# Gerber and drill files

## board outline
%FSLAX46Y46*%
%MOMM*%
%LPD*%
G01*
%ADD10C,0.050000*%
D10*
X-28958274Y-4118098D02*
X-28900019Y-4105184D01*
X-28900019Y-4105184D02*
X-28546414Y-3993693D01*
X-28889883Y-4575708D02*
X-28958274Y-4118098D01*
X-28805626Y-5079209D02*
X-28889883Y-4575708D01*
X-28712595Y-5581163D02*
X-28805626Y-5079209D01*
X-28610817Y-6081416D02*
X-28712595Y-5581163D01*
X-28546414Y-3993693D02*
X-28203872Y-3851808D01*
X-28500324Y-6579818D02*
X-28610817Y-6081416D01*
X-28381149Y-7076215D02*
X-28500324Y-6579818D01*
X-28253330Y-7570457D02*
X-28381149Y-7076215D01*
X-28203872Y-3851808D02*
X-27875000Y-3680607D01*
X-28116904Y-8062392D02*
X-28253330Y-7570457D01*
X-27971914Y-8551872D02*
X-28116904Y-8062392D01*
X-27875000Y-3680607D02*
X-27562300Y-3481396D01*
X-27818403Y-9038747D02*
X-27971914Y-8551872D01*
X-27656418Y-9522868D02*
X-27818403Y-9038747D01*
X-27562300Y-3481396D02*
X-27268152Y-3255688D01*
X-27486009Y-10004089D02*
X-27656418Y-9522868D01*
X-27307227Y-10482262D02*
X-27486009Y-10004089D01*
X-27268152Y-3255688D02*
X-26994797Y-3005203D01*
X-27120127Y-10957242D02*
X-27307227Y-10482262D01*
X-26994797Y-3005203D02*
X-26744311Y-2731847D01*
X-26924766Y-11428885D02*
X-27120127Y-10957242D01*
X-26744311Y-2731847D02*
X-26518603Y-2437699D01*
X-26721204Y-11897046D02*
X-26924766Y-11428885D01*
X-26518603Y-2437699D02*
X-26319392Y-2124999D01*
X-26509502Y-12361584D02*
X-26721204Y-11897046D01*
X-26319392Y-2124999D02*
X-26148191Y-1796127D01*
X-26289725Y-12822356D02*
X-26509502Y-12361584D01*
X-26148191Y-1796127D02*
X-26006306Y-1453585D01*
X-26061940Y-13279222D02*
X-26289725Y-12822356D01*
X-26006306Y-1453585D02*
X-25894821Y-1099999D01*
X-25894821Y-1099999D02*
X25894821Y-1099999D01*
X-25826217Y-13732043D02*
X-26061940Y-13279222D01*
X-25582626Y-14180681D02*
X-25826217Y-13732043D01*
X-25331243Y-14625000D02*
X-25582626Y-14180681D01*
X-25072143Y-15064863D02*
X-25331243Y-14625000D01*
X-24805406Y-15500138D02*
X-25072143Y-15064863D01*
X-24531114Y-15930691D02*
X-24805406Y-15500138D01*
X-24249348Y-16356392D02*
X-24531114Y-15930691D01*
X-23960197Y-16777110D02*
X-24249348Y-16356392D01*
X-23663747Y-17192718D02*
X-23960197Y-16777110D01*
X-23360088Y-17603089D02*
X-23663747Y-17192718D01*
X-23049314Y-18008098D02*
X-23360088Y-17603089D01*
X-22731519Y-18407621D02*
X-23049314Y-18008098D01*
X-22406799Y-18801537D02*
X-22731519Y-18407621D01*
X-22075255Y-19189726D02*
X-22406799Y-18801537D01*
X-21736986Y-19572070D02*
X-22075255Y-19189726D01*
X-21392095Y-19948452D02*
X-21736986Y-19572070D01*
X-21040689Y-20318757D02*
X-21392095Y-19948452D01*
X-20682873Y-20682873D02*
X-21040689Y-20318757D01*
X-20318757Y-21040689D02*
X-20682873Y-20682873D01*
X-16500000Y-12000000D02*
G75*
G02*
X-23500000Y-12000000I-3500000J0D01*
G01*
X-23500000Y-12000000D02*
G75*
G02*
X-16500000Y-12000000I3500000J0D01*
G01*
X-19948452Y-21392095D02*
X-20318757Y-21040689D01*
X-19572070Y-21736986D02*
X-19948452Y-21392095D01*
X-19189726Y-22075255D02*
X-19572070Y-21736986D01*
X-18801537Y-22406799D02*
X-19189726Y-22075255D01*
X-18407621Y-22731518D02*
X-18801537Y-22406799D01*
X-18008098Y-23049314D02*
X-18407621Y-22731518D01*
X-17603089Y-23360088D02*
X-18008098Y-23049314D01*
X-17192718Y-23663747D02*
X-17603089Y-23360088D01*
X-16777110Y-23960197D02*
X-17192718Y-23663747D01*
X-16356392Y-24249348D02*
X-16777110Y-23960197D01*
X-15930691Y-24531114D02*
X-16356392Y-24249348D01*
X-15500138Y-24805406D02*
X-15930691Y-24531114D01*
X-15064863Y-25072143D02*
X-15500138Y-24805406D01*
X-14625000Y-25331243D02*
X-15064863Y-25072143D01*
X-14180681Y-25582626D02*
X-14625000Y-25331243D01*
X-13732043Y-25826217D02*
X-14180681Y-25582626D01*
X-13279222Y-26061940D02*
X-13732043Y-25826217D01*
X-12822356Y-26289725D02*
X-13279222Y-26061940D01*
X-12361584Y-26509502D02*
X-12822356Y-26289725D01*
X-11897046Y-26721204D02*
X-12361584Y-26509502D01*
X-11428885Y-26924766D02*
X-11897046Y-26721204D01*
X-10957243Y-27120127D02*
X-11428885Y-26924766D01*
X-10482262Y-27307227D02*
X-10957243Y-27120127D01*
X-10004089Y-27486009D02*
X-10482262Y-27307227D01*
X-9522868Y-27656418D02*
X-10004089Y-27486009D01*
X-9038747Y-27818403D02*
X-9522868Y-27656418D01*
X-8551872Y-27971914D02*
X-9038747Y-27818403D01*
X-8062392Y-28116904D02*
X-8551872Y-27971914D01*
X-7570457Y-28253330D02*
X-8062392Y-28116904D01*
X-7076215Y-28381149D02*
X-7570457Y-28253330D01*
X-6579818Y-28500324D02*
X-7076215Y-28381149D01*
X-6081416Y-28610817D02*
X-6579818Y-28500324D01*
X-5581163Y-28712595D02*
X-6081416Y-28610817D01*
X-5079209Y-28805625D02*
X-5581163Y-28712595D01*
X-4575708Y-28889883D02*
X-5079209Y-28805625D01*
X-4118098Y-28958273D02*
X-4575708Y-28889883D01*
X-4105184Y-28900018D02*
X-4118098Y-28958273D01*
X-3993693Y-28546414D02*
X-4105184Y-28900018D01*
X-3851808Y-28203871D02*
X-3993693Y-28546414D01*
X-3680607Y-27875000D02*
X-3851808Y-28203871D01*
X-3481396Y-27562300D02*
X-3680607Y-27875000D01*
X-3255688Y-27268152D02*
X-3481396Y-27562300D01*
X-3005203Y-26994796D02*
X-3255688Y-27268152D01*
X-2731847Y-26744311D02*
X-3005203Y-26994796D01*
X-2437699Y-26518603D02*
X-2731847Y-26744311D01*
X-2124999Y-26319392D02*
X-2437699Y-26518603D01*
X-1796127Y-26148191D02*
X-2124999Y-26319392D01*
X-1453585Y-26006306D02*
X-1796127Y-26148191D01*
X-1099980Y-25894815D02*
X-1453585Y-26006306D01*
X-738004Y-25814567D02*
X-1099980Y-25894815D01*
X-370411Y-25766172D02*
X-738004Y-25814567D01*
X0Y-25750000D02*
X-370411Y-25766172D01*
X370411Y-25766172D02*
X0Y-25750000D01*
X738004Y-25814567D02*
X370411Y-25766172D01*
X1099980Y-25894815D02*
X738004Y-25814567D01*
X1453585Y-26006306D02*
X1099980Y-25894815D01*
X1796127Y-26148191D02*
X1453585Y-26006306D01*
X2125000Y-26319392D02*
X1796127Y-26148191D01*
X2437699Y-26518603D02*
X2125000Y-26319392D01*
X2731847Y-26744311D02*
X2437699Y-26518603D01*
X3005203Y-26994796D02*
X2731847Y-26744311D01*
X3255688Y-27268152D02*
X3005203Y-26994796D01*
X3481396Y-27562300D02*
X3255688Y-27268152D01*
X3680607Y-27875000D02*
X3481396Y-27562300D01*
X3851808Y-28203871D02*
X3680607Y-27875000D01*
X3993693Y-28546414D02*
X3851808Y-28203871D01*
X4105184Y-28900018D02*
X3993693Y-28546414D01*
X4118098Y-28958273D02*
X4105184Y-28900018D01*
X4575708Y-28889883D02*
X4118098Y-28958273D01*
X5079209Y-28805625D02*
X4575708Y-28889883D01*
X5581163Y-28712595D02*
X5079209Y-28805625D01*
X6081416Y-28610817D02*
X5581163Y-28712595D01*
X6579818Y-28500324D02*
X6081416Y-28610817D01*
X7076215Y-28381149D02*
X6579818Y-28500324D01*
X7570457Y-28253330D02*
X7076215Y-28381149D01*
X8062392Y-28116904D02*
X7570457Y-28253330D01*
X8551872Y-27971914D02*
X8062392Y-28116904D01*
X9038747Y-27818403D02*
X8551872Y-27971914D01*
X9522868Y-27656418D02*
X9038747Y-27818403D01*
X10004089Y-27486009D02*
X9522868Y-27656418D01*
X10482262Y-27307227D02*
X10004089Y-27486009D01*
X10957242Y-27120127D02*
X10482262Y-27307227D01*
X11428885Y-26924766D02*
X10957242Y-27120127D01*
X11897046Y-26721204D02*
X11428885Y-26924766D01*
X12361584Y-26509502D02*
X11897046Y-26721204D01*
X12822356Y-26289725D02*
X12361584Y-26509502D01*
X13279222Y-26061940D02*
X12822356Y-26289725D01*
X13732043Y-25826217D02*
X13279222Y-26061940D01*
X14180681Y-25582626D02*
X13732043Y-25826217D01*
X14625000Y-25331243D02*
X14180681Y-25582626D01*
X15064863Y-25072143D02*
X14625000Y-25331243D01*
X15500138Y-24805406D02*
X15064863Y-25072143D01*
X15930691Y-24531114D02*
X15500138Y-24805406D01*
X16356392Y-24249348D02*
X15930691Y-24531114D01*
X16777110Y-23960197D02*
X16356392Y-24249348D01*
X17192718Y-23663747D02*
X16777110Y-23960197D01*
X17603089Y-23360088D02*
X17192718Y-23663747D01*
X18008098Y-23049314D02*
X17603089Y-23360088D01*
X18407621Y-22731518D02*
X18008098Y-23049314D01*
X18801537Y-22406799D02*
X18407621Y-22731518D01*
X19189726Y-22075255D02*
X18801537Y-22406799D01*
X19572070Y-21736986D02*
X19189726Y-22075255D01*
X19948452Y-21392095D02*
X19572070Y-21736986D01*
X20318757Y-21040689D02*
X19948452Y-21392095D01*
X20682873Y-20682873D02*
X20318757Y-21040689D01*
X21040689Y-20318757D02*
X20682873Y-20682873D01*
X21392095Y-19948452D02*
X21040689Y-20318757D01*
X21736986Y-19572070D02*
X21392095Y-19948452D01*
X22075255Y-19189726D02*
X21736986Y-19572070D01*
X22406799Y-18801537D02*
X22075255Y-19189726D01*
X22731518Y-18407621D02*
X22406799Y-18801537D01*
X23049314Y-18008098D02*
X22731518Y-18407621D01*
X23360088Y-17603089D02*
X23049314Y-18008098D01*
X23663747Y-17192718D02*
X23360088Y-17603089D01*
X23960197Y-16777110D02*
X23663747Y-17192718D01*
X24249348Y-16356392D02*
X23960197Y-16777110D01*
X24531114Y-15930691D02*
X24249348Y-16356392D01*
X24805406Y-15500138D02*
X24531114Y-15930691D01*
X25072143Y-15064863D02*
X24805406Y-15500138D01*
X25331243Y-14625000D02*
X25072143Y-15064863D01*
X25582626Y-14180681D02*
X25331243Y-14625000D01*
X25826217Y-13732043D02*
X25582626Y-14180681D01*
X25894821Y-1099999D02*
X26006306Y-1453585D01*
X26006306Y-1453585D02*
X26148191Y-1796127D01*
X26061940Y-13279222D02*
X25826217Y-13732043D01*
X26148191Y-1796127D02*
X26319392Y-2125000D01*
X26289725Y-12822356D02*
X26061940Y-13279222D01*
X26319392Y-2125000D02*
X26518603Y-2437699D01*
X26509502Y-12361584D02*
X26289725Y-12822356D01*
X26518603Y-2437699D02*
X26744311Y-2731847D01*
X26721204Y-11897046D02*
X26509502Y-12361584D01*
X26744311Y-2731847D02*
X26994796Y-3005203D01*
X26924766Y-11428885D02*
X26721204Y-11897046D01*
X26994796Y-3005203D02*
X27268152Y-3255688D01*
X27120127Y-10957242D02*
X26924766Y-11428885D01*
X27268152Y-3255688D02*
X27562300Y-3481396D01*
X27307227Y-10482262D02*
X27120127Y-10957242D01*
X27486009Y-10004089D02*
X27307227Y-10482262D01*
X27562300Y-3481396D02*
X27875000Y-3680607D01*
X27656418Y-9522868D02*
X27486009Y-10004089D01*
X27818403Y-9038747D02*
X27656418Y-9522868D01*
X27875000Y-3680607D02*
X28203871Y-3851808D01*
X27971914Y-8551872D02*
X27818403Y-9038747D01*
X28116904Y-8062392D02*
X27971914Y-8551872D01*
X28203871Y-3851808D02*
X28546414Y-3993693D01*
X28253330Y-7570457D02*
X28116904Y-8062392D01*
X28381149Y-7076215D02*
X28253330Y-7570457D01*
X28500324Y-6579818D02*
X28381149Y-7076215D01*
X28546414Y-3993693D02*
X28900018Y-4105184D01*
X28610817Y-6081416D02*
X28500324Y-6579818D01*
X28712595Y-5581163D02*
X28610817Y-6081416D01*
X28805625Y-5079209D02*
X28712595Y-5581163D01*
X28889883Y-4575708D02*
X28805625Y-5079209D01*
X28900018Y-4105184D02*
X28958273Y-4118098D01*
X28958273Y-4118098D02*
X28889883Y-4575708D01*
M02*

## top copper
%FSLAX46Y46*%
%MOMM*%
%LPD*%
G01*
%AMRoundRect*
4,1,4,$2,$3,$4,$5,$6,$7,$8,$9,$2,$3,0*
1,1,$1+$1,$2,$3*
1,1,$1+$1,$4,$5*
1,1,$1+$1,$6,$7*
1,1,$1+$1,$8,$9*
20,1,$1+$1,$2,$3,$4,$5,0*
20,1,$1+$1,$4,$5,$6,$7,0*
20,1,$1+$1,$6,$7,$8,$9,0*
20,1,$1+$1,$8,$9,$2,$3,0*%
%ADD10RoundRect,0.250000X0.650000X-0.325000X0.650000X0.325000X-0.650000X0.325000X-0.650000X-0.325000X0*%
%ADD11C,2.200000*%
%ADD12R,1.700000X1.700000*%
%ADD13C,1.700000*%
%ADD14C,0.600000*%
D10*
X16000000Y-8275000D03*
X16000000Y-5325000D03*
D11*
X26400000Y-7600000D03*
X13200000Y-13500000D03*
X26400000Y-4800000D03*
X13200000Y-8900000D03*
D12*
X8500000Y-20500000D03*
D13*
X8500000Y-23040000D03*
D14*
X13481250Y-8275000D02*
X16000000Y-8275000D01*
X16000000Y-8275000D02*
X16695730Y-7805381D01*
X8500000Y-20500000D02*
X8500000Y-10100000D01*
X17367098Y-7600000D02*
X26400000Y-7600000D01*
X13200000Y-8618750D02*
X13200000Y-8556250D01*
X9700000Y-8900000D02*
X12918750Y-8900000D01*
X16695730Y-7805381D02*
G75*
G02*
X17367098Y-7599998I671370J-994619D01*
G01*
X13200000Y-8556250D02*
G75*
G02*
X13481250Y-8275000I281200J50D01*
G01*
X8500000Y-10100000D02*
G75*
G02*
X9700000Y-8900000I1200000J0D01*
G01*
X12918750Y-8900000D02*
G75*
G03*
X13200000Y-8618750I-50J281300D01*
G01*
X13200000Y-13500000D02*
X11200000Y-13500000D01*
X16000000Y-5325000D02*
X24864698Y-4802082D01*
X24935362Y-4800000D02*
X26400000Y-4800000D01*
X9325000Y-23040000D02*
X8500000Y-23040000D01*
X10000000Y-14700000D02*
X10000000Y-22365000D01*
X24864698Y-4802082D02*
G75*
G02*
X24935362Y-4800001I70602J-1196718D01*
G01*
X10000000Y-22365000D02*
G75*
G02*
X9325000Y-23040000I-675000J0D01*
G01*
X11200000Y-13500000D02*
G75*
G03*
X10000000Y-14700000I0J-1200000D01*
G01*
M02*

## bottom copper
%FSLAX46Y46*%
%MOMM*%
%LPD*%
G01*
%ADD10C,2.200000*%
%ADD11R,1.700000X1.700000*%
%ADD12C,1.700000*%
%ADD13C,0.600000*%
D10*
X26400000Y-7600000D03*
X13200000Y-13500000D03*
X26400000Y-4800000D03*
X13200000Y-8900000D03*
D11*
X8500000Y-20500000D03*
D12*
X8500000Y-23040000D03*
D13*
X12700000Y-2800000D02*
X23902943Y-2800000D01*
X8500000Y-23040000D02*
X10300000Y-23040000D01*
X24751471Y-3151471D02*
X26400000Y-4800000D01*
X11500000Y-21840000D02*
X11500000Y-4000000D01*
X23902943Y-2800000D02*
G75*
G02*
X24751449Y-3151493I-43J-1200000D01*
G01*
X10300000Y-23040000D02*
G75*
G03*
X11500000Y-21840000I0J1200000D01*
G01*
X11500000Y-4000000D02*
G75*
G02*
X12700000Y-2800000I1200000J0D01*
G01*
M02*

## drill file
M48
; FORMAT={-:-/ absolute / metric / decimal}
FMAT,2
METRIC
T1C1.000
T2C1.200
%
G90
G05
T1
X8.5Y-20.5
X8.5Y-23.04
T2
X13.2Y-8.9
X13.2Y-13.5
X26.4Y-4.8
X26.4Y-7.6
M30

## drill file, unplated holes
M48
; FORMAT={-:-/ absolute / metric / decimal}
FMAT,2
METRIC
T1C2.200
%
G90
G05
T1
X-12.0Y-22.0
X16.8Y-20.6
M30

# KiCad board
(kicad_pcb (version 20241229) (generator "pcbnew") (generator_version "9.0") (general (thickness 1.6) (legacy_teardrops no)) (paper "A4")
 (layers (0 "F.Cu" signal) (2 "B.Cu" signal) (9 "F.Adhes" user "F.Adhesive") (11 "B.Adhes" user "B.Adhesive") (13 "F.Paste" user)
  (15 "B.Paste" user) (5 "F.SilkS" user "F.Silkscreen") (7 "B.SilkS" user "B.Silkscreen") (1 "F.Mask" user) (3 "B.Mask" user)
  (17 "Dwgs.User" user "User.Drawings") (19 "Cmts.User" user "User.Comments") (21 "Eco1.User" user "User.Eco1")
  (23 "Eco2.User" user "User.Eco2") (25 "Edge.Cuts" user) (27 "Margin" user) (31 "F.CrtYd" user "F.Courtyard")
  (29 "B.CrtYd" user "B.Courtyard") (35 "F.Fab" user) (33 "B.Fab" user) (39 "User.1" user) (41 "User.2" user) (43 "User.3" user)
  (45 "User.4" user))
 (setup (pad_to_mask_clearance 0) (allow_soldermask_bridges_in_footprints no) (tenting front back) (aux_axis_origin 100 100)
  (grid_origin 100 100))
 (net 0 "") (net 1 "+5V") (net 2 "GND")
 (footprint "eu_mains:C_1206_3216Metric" (layer "F.Cu") (at 116 106.8 90)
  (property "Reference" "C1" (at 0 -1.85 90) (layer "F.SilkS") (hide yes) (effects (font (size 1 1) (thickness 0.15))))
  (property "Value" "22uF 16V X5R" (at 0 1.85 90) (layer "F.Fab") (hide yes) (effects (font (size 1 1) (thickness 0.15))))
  (pad "1" smd roundrect (at -1.475 0 90) (size 1.15 1.8) (layers "F.Cu" "F.Mask" "F.Paste") (roundrect_rratio 0.217391) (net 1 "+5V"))
  (pad "2" smd roundrect (at 1.475 0 90) (size 1.15 1.8) (layers "F.Cu" "F.Mask" "F.Paste") (roundrect_rratio 0.217391) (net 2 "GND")))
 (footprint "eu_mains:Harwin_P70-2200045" (layer "F.Cu") (at 126.4 107.6)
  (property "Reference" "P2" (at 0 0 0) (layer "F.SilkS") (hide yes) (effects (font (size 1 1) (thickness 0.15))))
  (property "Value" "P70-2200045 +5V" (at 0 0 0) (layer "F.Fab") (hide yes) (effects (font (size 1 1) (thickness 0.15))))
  (pad "1" thru_hole circle (at 0 0) (size 2.2 2.2) (drill 1.2) (layers "*.Cu" "*.Mask" "F.Paste") (remove_unused_layers no) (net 1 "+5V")))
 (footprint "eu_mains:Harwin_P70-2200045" (layer "F.Cu") (at 113.2 113.5)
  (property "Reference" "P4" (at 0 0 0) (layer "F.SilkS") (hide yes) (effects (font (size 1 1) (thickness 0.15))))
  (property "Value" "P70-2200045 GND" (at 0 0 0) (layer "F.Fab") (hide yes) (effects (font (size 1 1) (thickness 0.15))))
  (pad "1" thru_hole circle (at 0 0) (size 2.2 2.2) (drill 1.2) (layers "*.Cu" "*.Mask" "F.Paste") (remove_unused_layers no) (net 2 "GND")))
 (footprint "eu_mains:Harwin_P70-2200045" (layer "F.Cu") (at 126.4 104.8)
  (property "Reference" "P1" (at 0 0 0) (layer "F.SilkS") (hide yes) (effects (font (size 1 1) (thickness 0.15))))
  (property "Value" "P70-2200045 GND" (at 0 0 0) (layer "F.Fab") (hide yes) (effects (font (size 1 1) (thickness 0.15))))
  (pad "1" thru_hole circle (at 0 0) (size 2.2 2.2) (drill 1.2) (layers "*.Cu" "*.Mask" "F.Paste") (remove_unused_layers no) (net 2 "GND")))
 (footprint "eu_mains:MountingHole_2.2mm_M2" (layer "F.Cu") (at 116.8 120.6)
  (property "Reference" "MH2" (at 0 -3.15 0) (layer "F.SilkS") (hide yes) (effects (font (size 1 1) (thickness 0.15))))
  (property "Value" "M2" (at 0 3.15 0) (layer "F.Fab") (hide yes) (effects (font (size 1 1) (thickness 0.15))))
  (pad "" np_thru_hole circle (at 0 0) (size 2.2 2.2) (drill 2.2) (layers "*.Cu" "*.Mask")))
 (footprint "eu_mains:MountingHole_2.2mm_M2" (layer "F.Cu") (at 88 122)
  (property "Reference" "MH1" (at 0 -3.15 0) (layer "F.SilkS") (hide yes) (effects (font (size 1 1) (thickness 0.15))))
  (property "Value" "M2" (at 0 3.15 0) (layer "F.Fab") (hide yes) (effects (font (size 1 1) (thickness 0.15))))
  (pad "" np_thru_hole circle (at 0 0) (size 2.2 2.2) (drill 2.2) (layers "*.Cu" "*.Mask")))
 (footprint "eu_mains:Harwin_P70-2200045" (layer "F.Cu") (at 113.2 108.9)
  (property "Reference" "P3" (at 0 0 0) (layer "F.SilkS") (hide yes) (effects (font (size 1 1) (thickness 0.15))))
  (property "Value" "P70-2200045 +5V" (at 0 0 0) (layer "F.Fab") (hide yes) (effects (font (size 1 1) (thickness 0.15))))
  (pad "1" thru_hole circle (at 0 0) (size 2.2 2.2) (drill 1.2) (layers "*.Cu" "*.Mask" "F.Paste") (remove_unused_layers no) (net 1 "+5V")))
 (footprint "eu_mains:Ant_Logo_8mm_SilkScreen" (layer "F.Cu") (at 90.1 106.7)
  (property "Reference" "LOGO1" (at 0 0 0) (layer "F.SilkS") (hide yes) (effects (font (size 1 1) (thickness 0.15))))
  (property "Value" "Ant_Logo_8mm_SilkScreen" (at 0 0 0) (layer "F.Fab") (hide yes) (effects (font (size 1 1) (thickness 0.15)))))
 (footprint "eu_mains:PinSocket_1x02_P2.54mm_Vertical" (layer "B.Cu") (at 108.5 120.5 180)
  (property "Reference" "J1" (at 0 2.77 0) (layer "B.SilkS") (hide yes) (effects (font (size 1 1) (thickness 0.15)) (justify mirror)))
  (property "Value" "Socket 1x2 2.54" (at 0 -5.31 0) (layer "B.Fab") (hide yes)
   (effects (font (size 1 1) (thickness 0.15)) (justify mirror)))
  (pad "1" thru_hole rect (at 0 0 180) (size 1.7 1.7) (drill 1) (layers "*.Cu" "*.Mask") (remove_unused_layers no) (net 1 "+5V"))
  (pad "2" thru_hole circle (at 0 -2.54 180) (size 1.7 1.7) (drill 1) (layers "*.Cu" "*.Mask") (remove_unused_layers no) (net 2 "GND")))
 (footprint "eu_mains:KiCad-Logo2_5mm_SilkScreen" (layer "B.Cu") (at 102.4 105.7 180)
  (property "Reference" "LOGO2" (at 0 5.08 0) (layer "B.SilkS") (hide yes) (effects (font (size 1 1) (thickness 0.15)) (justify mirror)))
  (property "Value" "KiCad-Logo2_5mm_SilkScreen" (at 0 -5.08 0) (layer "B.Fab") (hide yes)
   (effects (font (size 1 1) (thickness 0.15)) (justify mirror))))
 (gr_line (start 71.041726 104.118098) (end 71.099981 104.105184) (stroke (width 0.05) (type default)) (layer "Edge.Cuts"))
 (gr_line (start 71.099981 104.105184) (end 71.453586 103.993693) (stroke (width 0.05) (type default)) (layer "Edge.Cuts"))
 (gr_line (start 71.110117 104.575708) (end 71.041726 104.118098) (stroke (width 0.05) (type default)) (layer "Edge.Cuts"))
 (gr_line (start 71.194374 105.079209) (end 71.110117 104.575708) (stroke (width 0.05) (type default)) (layer "Edge.Cuts"))
 (gr_line (start 71.287405 105.581163) (end 71.194374 105.079209) (stroke (width 0.05) (type default)) (layer "Edge.Cuts"))
 (gr_line (start 71.389183 106.081416) (end 71.287405 105.581163) (stroke (width 0.05) (type default)) (layer "Edge.Cuts"))
 (gr_line (start 71.453586 103.993693) (end 71.796128 103.851808) (stroke (width 0.05) (type default)) (layer "Edge.Cuts"))
 (gr_line (start 71.499676 106.579818) (end 71.389183 106.081416) (stroke (width 0.05) (type default)) (layer "Edge.Cuts"))
 (gr_line (start 71.618851 107.076215) (end 71.499676 106.579818) (stroke (width 0.05) (type default)) (layer "Edge.Cuts"))
 (gr_line (start 71.74667 107.570457) (end 71.618851 107.076215) (stroke (width 0.05) (type default)) (layer "Edge.Cuts"))
 (gr_line (start 71.796128 103.851808) (end 72.125 103.680607) (stroke (width 0.05) (type default)) (layer "Edge.Cuts"))
 (gr_line (start 71.883096 108.062392) (end 71.74667 107.570457) (stroke (width 0.05) (type default)) (layer "Edge.Cuts"))
 (gr_line (start 72.028086 108.551872) (end 71.883096 108.062392) (stroke (width 0.05) (type default)) (layer "Edge.Cuts"))
 (gr_line (start 72.125 103.680607) (end 72.4377 103.481396) (stroke (width 0.05) (type default)) (layer "Edge.Cuts"))
 (gr_line (start 72.181597 109.038747) (end 72.028086 108.551872) (stroke (width 0.05) (type default)) (layer "Edge.Cuts"))
 (gr_line (start 72.343582 109.522868) (end 72.181597 109.038747) (stroke (width 0.05) (type default)) (layer "Edge.Cuts"))
 (gr_line (start 72.4377 103.481396) (end 72.731848 103.255688) (stroke (width 0.05) (type default)) (layer "Edge.Cuts"))
 (gr_line (start 72.513991 110.004089) (end 72.343582 109.522868) (stroke (width 0.05) (type default)) (layer "Edge.Cuts"))
 (gr_line (start 72.692773 110.482262) (end 72.513991 110.004089) (stroke (width 0.05) (type default)) (layer "Edge.Cuts"))
 (gr_line (start 72.731848 103.255688) (end 73.005203 103.005203) (stroke (width 0.05) (type default)) (layer "Edge.Cuts"))
 (gr_line (start 72.879873 110.957242) (end 72.692773 110.482262) (stroke (width 0.05) (type default)) (layer "Edge.Cuts"))
 (gr_line (start 73.005203 103.005203) (end 73.255689 102.731847) (stroke (width 0.05) (type default)) (layer "Edge.Cuts"))
 (gr_line (start 73.075234 111.428885) (end 72.879873 110.957242) (stroke (width 0.05) (type default)) (layer "Edge.Cuts"))
 (gr_line (start 73.255689 102.731847) (end 73.481397 102.437699) (stroke (width 0.05) (type default)) (layer "Edge.Cuts"))
 (gr_line (start 73.278796 111.897046) (end 73.075234 111.428885) (stroke (width 0.05) (type default)) (layer "Edge.Cuts"))
 (gr_line (start 73.481397 102.437699) (end 73.680608 102.124999) (stroke (width 0.05) (type default)) (layer "Edge.Cuts"))
 (gr_line (start 73.490498 112.361584) (end 73.278796 111.897046) (stroke (width 0.05) (type default)) (layer "Edge.Cuts"))
 (gr_line (start 73.680608 102.124999) (end 73.851809 101.796127) (stroke (width 0.05) (type default)) (layer "Edge.Cuts"))
 (gr_line (start 73.710275 112.822356) (end 73.490498 112.361584) (stroke (width 0.05) (type default)) (layer "Edge.Cuts"))
 (gr_line (start 73.851809 101.796127) (end 73.993694 101.453585) (stroke (width 0.05) (type default)) (layer "Edge.Cuts"))
 (gr_line (start 73.93806 113.279222) (end 73.710275 112.822356) (stroke (width 0.05) (type default)) (layer "Edge.Cuts"))
 (gr_line (start 73.993694 101.453585) (end 74.105179 101.099999) (stroke (width 0.05) (type default)) (layer "Edge.Cuts"))
 (gr_line (start 74.105179 101.099999) (end 125.894821 101.099999) (stroke (width 0.05) (type default)) (layer "Edge.Cuts"))
 (gr_line (start 74.173783 113.732043) (end 73.93806 113.279222) (stroke (width 0.05) (type default)) (layer "Edge.Cuts"))
 (gr_line (start 74.417374 114.180681) (end 74.173783 113.732043) (stroke (width 0.05) (type default)) (layer "Edge.Cuts"))
 (gr_line (start 74.668757 114.625) (end 74.417374 114.180681) (stroke (width 0.05) (type default)) (layer "Edge.Cuts"))
 (gr_line (start 74.927857 115.064863) (end 74.668757 114.625) (stroke (width 0.05) (type default)) (layer "Edge.Cuts"))
 (gr_line (start 75.194594 115.500138) (end 74.927857 115.064863) (stroke (width 0.05) (type default)) (layer "Edge.Cuts"))
 (gr_line (start 75.468886 115.930691) (end 75.194594 115.500138) (stroke (width 0.05) (type default)) (layer "Edge.Cuts"))
 (gr_line (start 75.750652 116.356392) (end 75.468886 115.930691) (stroke (width 0.05) (type default)) (layer "Edge.Cuts"))
 (gr_line (start 76.039803 116.77711) (end 75.750652 116.356392) (stroke (width 0.05) (type default)) (layer "Edge.Cuts"))
 (gr_line (start 76.336253 117.192718) (end 76.039803 116.77711) (stroke (width 0.05) (type default)) (layer "Edge.Cuts"))
 (gr_line (start 76.639912 117.603089) (end 76.336253 117.192718) (stroke (width 0.05) (type default)) (layer "Edge.Cuts"))
 (gr_line (start 76.950686 118.008098) (end 76.639912 117.603089) (stroke (width 0.05) (type default)) (layer "Edge.Cuts"))
 (gr_line (start 77.268481 118.407621) (end 76.950686 118.008098) (stroke (width 0.05) (type default)) (layer "Edge.Cuts"))
 (gr_line (start 77.593201 118.801537) (end 77.268481 118.407621) (stroke (width 0.05) (type default)) (layer "Edge.Cuts"))
 (gr_line (start 77.924745 119.189726) (end 77.593201 118.801537) (stroke (width 0.05) (type default)) (layer "Edge.Cuts"))
 (gr_line (start 78.263014 119.57207) (end 77.924745 119.189726) (stroke (width 0.05) (type default)) (layer "Edge.Cuts"))
 (gr_line (start 78.607905 119.948452) (end 78.263014 119.57207) (stroke (width 0.05) (type default)) (layer "Edge.Cuts"))
 (gr_line (start 78.959311 120.318757) (end 78.607905 119.948452) (stroke (width 0.05) (type default)) (layer "Edge.Cuts"))
 (gr_line (start 79.317127 120.682873) (end 78.959311 120.318757) (stroke (width 0.05) (type default)) (layer "Edge.Cuts"))
 (gr_line (start 79.681243 121.040689) (end 79.317127 120.682873) (stroke (width 0.05) (type default)) (layer "Edge.Cuts"))
 (gr_circle (center 80 112) (end 83.5 112) (stroke (width 0.05) (type default)) (fill no) (layer "Edge.Cuts"))
 (gr_line (start 80.051548 121.392095) (end 79.681243 121.040689) (stroke (width 0.05) (type default)) (layer "Edge.Cuts"))
 (gr_line (start 80.42793 121.736986) (end 80.051548 121.392095) (stroke (width 0.05) (type default)) (layer "Edge.Cuts"))
 (gr_line (start 80.810274 122.075255) (end 80.42793 121.736986) (stroke (width 0.05) (type default)) (layer "Edge.Cuts"))
 (gr_line (start 81.198463 122.406799) (end 80.810274 122.075255) (stroke (width 0.05) (type default)) (layer "Edge.Cuts"))
 (gr_line (start 81.592379 122.731518) (end 81.198463 122.406799) (stroke (width 0.05) (type default)) (layer "Edge.Cuts"))
 (gr_line (start 81.991902 123.049314) (end 81.592379 122.731518) (stroke (width 0.05) (type default)) (layer "Edge.Cuts"))
 (gr_line (start 82.396911 123.360088) (end 81.991902 123.049314) (stroke (width 0.05) (type default)) (layer "Edge.Cuts"))
 (gr_line (start 82.807282 123.663747) (end 82.396911 123.360088) (stroke (width 0.05) (type default)) (layer "Edge.Cuts"))
 (gr_line (start 83.22289 123.960197) (end 82.807282 123.663747) (stroke (width 0.05) (type default)) (layer "Edge.Cuts"))
 (gr_line (start 83.643608 124.249348) (end 83.22289 123.960197) (stroke (width 0.05) (type default)) (layer "Edge.Cuts"))
 (gr_line (start 84.069309 124.531114) (end 83.643608 124.249348) (stroke (width 0.05) (type default)) (layer "Edge.Cuts"))
 (gr_line (start 84.499862 124.805406) (end 84.069309 124.531114) (stroke (width 0.05) (type default)) (layer "Edge.Cuts"))
 (gr_line (start 84.935137 125.072143) (end 84.499862 124.805406) (stroke (width 0.05) (type default)) (layer "Edge.Cuts"))
 (gr_line (start 85.375 125.331243) (end 84.935137 125.072143) (stroke (width 0.05) (type default)) (layer "Edge.Cuts"))
 (gr_line (start 85.819319 125.582626) (end 85.375 125.331243) (stroke (width 0.05) (type default)) (layer "Edge.Cuts"))
 (gr_line (start 86.267957 125.826217) (end 85.819319 125.582626) (stroke (width 0.05) (type default)) (layer "Edge.Cuts"))
 (gr_line (start 86.720778 126.06194) (end 86.267957 125.826217) (stroke (width 0.05) (type default)) (layer "Edge.Cuts"))
 (gr_line (start 87.177644 126.289725) (end 86.720778 126.06194) (stroke (width 0.05) (type default)) (layer "Edge.Cuts"))
 (gr_line (start 87.638416 126.509502) (end 87.177644 126.289725) (stroke (width 0.05) (type default)) (layer "Edge.Cuts"))
 (gr_line (start 88.102954 126.721204) (end 87.638416 126.509502) (stroke (width 0.05) (type default)) (layer "Edge.Cuts"))
 (gr_line (start 88.571115 126.924766) (end 88.102954 126.721204) (stroke (width 0.05) (type default)) (layer "Edge.Cuts"))
 (gr_line (start 89.042757 127.120127) (end 88.571115 126.924766) (stroke (width 0.05) (type default)) (layer "Edge.Cuts"))
 (gr_line (start 89.517738 127.307227) (end 89.042757 127.120127) (stroke (width 0.05) (type default)) (layer "Edge.Cuts"))
 (gr_line (start 89.995911 127.486009) (end 89.517738 127.307227) (stroke (width 0.05) (type default)) (layer "Edge.Cuts"))
 (gr_line (start 90.477132 127.656418) (end 89.995911 127.486009) (stroke (width 0.05) (type default)) (layer "Edge.Cuts"))
 (gr_line (start 90.961253 127.818403) (end 90.477132 127.656418) (stroke (width 0.05) (type default)) (layer "Edge.Cuts"))
 (gr_line (start 91.448128 127.971914) (end 90.961253 127.818403) (stroke (width 0.05) (type default)) (layer "Edge.Cuts"))
 (gr_line (start 91.937608 128.116904) (end 91.448128 127.971914) (stroke (width 0.05) (type default)) (layer "Edge.Cuts"))
 (gr_line (start 92.429543 128.25333) (end 91.937608 128.116904) (stroke (width 0.05) (type default)) (layer "Edge.Cuts"))
 (gr_line (start 92.923785 128.381149) (end 92.429543 128.25333) (stroke (width 0.05) (type default)) (layer "Edge.Cuts"))
 (gr_line (start 93.420182 128.500324) (end 92.923785 128.381149) (stroke (width 0.05) (type default)) (layer "Edge.Cuts"))
 (gr_line (start 93.918584 128.610817) (end 93.420182 128.500324) (stroke (width 0.05) (type default)) (layer "Edge.Cuts"))
 (gr_line (start 94.418837 128.712595) (end 93.918584 128.610817) (stroke (width 0.05) (type default)) (layer "Edge.Cuts"))
 (gr_line (start 94.920791 128.805625) (end 94.418837 128.712595) (stroke (width 0.05) (type default)) (layer "Edge.Cuts"))
 (gr_line (start 95.424292 128.889883) (end 94.920791 128.805625) (stroke (width 0.05) (type default)) (layer "Edge.Cuts"))
 (gr_line (start 95.881902 128.958273) (end 95.424292 128.889883) (stroke (width 0.05) (type default)) (layer "Edge.Cuts"))
 (gr_line (start 95.894816 128.900018) (end 95.881902 128.958273) (stroke (width 0.05) (type default)) (layer "Edge.Cuts"))
 (gr_line (start 96.006307 128.546414) (end 95.894816 128.900018) (stroke (width 0.05) (type default)) (layer "Edge.Cuts"))
 (gr_line (start 96.148192 128.203871) (end 96.006307 128.546414) (stroke (width 0.05) (type default)) (layer "Edge.Cuts"))
 (gr_line (start 96.319393 127.875) (end 96.148192 128.203871) (stroke (width 0.05) (type default)) (layer "Edge.Cuts"))
 (gr_line (start 96.518604 127.5623) (end 96.319393 127.875) (stroke (width 0.05) (type default)) (layer "Edge.Cuts"))
 (gr_line (start 96.744312 127.268152) (end 96.518604 127.5623) (stroke (width 0.05) (type default)) (layer "Edge.Cuts"))
 (gr_line (start 96.994797 126.994796) (end 96.744312 127.268152) (stroke (width 0.05) (type default)) (layer "Edge.Cuts"))
 (gr_line (start 97.268153 126.744311) (end 96.994797 126.994796) (stroke (width 0.05) (type default)) (layer "Edge.Cuts"))
 (gr_line (start 97.562301 126.518603) (end 97.268153 126.744311) (stroke (width 0.05) (type default)) (layer "Edge.Cuts"))
 (gr_line (start 97.875001 126.319392) (end 97.562301 126.518603) (stroke (width 0.05) (type default)) (layer "Edge.Cuts"))
 (gr_line (start 98.203873 126.148191) (end 97.875001 126.319392) (stroke (width 0.05) (type default)) (layer "Edge.Cuts"))
 (gr_line (start 98.546415 126.006306) (end 98.203873 126.148191) (stroke (width 0.05) (type default)) (layer "Edge.Cuts"))
 (gr_line (start 98.90002 125.894815) (end 98.546415 126.006306) (stroke (width 0.05) (type default)) (layer "Edge.Cuts"))
 (gr_line (start 99.261996 125.814567) (end 98.90002 125.894815) (stroke (width 0.05) (type default)) (layer "Edge.Cuts"))
 (gr_line (start 99.629589 125.766172) (end 99.261996 125.814567) (stroke (width 0.05) (type default)) (layer "Edge.Cuts"))
 (gr_line (start 100 125.75) (end 99.629589 125.766172) (stroke (width 0.05) (type default)) (layer "Edge.Cuts"))
 (gr_line (start 100.370411 125.766172) (end 100 125.75) (stroke (width 0.05) (type default)) (layer "Edge.Cuts"))
 (gr_line (start 100.738004 125.814567) (end 100.370411 125.766172) (stroke (width 0.05) (type default)) (layer "Edge.Cuts"))
 (gr_line (start 101.09998 125.894815) (end 100.738004 125.814567) (stroke (width 0.05) (type default)) (layer "Edge.Cuts"))
 (gr_line (start 101.453585 126.006306) (end 101.09998 125.894815) (stroke (width 0.05) (type default)) (layer "Edge.Cuts"))
 (gr_line (start 101.796127 126.148191) (end 101.453585 126.006306) (stroke (width 0.05) (type default)) (layer "Edge.Cuts"))
 (gr_line (start 102.125 126.319392) (end 101.796127 126.148191) (stroke (width 0.05) (type default)) (layer "Edge.Cuts"))
 (gr_line (start 102.437699 126.518603) (end 102.125 126.319392) (stroke (width 0.05) (type default)) (layer "Edge.Cuts"))
 (gr_line (start 102.731847 126.744311) (end 102.437699 126.518603) (stroke (width 0.05) (type default)) (layer "Edge.Cuts"))
 (gr_line (start 103.005203 126.994796) (end 102.731847 126.744311) (stroke (width 0.05) (type default)) (layer "Edge.Cuts"))
 (gr_line (start 103.255688 127.268152) (end 103.005203 126.994796) (stroke (width 0.05) (type default)) (layer "Edge.Cuts"))
 (gr_line (start 103.481396 127.5623) (end 103.255688 127.268152) (stroke (width 0.05) (type default)) (layer "Edge.Cuts"))
 (gr_line (start 103.680607 127.875) (end 103.481396 127.5623) (stroke (width 0.05) (type default)) (layer "Edge.Cuts"))
 (gr_line (start 103.851808 128.203871) (end 103.680607 127.875) (stroke (width 0.05) (type default)) (layer "Edge.Cuts"))
 (gr_line (start 103.993693 128.546414) (end 103.851808 128.203871) (stroke (width 0.05) (type default)) (layer "Edge.Cuts"))
 (gr_line (start 104.105184 128.900018) (end 103.993693 128.546414) (stroke (width 0.05) (type default)) (layer "Edge.Cuts"))
 (gr_line (start 104.118098 128.958273) (end 104.105184 128.900018) (stroke (width 0.05) (type default)) (layer "Edge.Cuts"))
 (gr_line (start 104.575708 128.889883) (end 104.118098 128.958273) (stroke (width 0.05) (type default)) (layer "Edge.Cuts"))
 (gr_line (start 105.079209 128.805625) (end 104.575708 128.889883) (stroke (width 0.05) (type default)) (layer "Edge.Cuts"))
 (gr_line (start 105.581163 128.712595) (end 105.079209 128.805625) (stroke (width 0.05) (type default)) (layer "Edge.Cuts"))
 (gr_line (start 106.081416 128.610817) (end 105.581163 128.712595) (stroke (width 0.05) (type default)) (layer "Edge.Cuts"))
 (gr_line (start 106.579818 128.500324) (end 106.081416 128.610817) (stroke (width 0.05) (type default)) (layer "Edge.Cuts"))
 (gr_line (start 107.076215 128.381149) (end 106.579818 128.500324) (stroke (width 0.05) (type default)) (layer "Edge.Cuts"))
 (gr_line (start 107.570457 128.25333) (end 107.076215 128.381149) (stroke (width 0.05) (type default)) (layer "Edge.Cuts"))
 (gr_line (start 108.062392 128.116904) (end 107.570457 128.25333) (stroke (width 0.05) (type default)) (layer "Edge.Cuts"))
 (gr_line (start 108.551872 127.971914) (end 108.062392 128.116904) (stroke (width 0.05) (type default)) (layer "Edge.Cuts"))
 (gr_line (start 109.038747 127.818403) (end 108.551872 127.971914) (stroke (width 0.05) (type default)) (layer "Edge.Cuts"))
 (gr_line (start 109.522868 127.656418) (end 109.038747 127.818403) (stroke (width 0.05) (type default)) (layer "Edge.Cuts"))
 (gr_line (start 110.004089 127.486009) (end 109.522868 127.656418) (stroke (width 0.05) (type default)) (layer "Edge.Cuts"))
 (gr_line (start 110.482262 127.307227) (end 110.004089 127.486009) (stroke (width 0.05) (type default)) (layer "Edge.Cuts"))
 (gr_line (start 110.957242 127.120127) (end 110.482262 127.307227) (stroke (width 0.05) (type default)) (layer "Edge.Cuts"))
 (gr_line (start 111.428885 126.924766) (end 110.957242 127.120127) (stroke (width 0.05) (type default)) (layer "Edge.Cuts"))
 (gr_line (start 111.897046 126.721204) (end 111.428885 126.924766) (stroke (width 0.05) (type default)) (layer "Edge.Cuts"))
 (gr_line (start 112.361584 126.509502) (end 111.897046 126.721204) (stroke (width 0.05) (type default)) (layer "Edge.Cuts"))
 (gr_line (start 112.822356 126.289725) (end 112.361584 126.509502) (stroke (width 0.05) (type default)) (layer "Edge.Cuts"))
 (gr_line (start 113.279222 126.06194) (end 112.822356 126.289725) (stroke (width 0.05) (type default)) (layer "Edge.Cuts"))
 (gr_line (start 113.732043 125.826217) (end 113.279222 126.06194) (stroke (width 0.05) (type default)) (layer "Edge.Cuts"))
 (gr_line (start 114.180681 125.582626) (end 113.732043 125.826217) (stroke (width 0.05) (type default)) (layer "Edge.Cuts"))
 (gr_line (start 114.625 125.331243) (end 114.180681 125.582626) (stroke (width 0.05) (type default)) (layer "Edge.Cuts"))
 (gr_line (start 115.064863 125.072143) (end 114.625 125.331243) (stroke (width 0.05) (type default)) (layer "Edge.Cuts"))
 (gr_line (start 115.500138 124.805406) (end 115.064863 125.072143) (stroke (width 0.05) (type default)) (layer "Edge.Cuts"))
 (gr_line (start 115.930691 124.531114) (end 115.500138 124.805406) (stroke (width 0.05) (type default)) (layer "Edge.Cuts"))
 (gr_line (start 116.356392 124.249348) (end 115.930691 124.531114) (stroke (width 0.05) (type default)) (layer "Edge.Cuts"))
 (gr_line (start 116.77711 123.960197) (end 116.356392 124.249348) (stroke (width 0.05) (type default)) (layer "Edge.Cuts"))
 (gr_line (start 117.192718 123.663747) (end 116.77711 123.960197) (stroke (width 0.05) (type default)) (layer "Edge.Cuts"))
 (gr_line (start 117.603089 123.360088) (end 117.192718 123.663747) (stroke (width 0.05) (type default)) (layer "Edge.Cuts"))
 (gr_line (start 118.008098 123.049314) (end 117.603089 123.360088) (stroke (width 0.05) (type default)) (layer "Edge.Cuts"))
 (gr_line (start 118.407621 122.731518) (end 118.008098 123.049314) (stroke (width 0.05) (type default)) (layer "Edge.Cuts"))
 (gr_line (start 118.801537 122.406799) (end 118.407621 122.731518) (stroke (width 0.05) (type default)) (layer "Edge.Cuts"))
 (gr_line (start 119.189726 122.075255) (end 118.801537 122.406799) (stroke (width 0.05) (type default)) (layer "Edge.Cuts"))
 (gr_line (start 119.57207 121.736986) (end 119.189726 122.075255) (stroke (width 0.05) (type default)) (layer "Edge.Cuts"))
 (gr_line (start 119.948452 121.392095) (end 119.57207 121.736986) (stroke (width 0.05) (type default)) (layer "Edge.Cuts"))
 (gr_line (start 120.318757 121.040689) (end 119.948452 121.392095) (stroke (width 0.05) (type default)) (layer "Edge.Cuts"))
 (gr_line (start 120.682873 120.682873) (end 120.318757 121.040689) (stroke (width 0.05) (type default)) (layer "Edge.Cuts"))
 (gr_line (start 121.040689 120.318757) (end 120.682873 120.682873) (stroke (width 0.05) (type default)) (layer "Edge.Cuts"))
 (gr_line (start 121.392095 119.948452) (end 121.040689 120.318757) (stroke (width 0.05) (type default)) (layer "Edge.Cuts"))
 (gr_line (start 121.736986 119.57207) (end 121.392095 119.948452) (stroke (width 0.05) (type default)) (layer "Edge.Cuts"))
 (gr_line (start 122.075255 119.189726) (end 121.736986 119.57207) (stroke (width 0.05) (type default)) (layer "Edge.Cuts"))
 (gr_line (start 122.406799 118.801537) (end 122.075255 119.189726) (stroke (width 0.05) (type default)) (layer "Edge.Cuts"))
 (gr_line (start 122.731518 118.407621) (end 122.406799 118.801537) (stroke (width 0.05) (type default)) (layer "Edge.Cuts"))
 (gr_line (start 123.049314 118.008098) (end 122.731518 118.407621) (stroke (width 0.05) (type default)) (layer "Edge.Cuts"))
 (gr_line (start 123.360088 117.603089) (end 123.049314 118.008098) (stroke (width 0.05) (type default)) (layer "Edge.Cuts"))
 (gr_line (start 123.663747 117.192718) (end 123.360088 117.603089) (stroke (width 0.05) (type default)) (layer "Edge.Cuts"))
 (gr_line (start 123.960197 116.77711) (end 123.663747 117.192718) (stroke (width 0.05) (type default)) (layer "Edge.Cuts"))
 (gr_line (start 124.249348 116.356392) (end 123.960197 116.77711) (stroke (width 0.05) (type default)) (layer "Edge.Cuts"))
 (gr_line (start 124.531114 115.930691) (end 124.249348 116.356392) (stroke (width 0.05) (type default)) (layer "Edge.Cuts"))
 (gr_line (start 124.805406 115.500138) (end 124.531114 115.930691) (stroke (width 0.05) (type default)) (layer "Edge.Cuts"))
 (gr_line (start 125.072143 115.064863) (end 124.805406 115.500138) (stroke (width 0.05) (type default)) (layer "Edge.Cuts"))
 (gr_line (start 125.331243 114.625) (end 125.072143 115.064863) (stroke (width 0.05) (type default)) (layer "Edge.Cuts"))
 (gr_line (start 125.582626 114.180681) (end 125.331243 114.625) (stroke (width 0.05) (type default)) (layer "Edge.Cuts"))
 (gr_line (start 125.826217 113.732043) (end 125.582626 114.180681) (stroke (width 0.05) (type default)) (layer "Edge.Cuts"))
 (gr_line (start 125.894821 101.099999) (end 126.006306 101.453585) (stroke (width 0.05) (type default)) (layer "Edge.Cuts"))
 (gr_line (start 126.006306 101.453585) (end 126.148191 101.796127) (stroke (width 0.05) (type default)) (layer "Edge.Cuts"))
 (gr_line (start 126.06194 113.279222) (end 125.826217 113.732043) (stroke (width 0.05) (type default)) (layer "Edge.Cuts"))
 (gr_line (start 126.148191 101.796127) (end 126.319392 102.125) (stroke (width 0.05) (type default)) (layer "Edge.Cuts"))
 (gr_line (start 126.289725 112.822356) (end 126.06194 113.279222) (stroke (width 0.05) (type default)) (layer "Edge.Cuts"))
 (gr_line (start 126.319392 102.125) (end 126.518603 102.437699) (stroke (width 0.05) (type default)) (layer "Edge.Cuts"))
 (gr_line (start 126.509502 112.361584) (end 126.289725 112.822356) (stroke (width 0.05) (type default)) (layer "Edge.Cuts"))
 (gr_line (start 126.518603 102.437699) (end 126.744311 102.731847) (stroke (width 0.05) (type default)) (layer "Edge.Cuts"))
 (gr_line (start 126.721204 111.897046) (end 126.509502 112.361584) (stroke (width 0.05) (type default)) (layer "Edge.Cuts"))
 (gr_line (start 126.744311 102.731847) (end 126.994796 103.005203) (stroke (width 0.05) (type default)) (layer "Edge.Cuts"))
 (gr_line (start 126.924766 111.428885) (end 126.721204 111.897046) (stroke (width 0.05) (type default)) (layer "Edge.Cuts"))
 (gr_line (start 126.994796 103.005203) (end 127.268152 103.255688) (stroke (width 0.05) (type default)) (layer "Edge.Cuts"))
 (gr_line (start 127.120127 110.957242) (end 126.924766 111.428885) (stroke (width 0.05) (type default)) (layer "Edge.Cuts"))
 (gr_line (start 127.268152 103.255688) (end 127.5623 103.481396) (stroke (width 0.05) (type default)) (layer "Edge.Cuts"))
 (gr_line (start 127.307227 110.482262) (end 127.120127 110.957242) (stroke (width 0.05) (type default)) (layer "Edge.Cuts"))
 (gr_line (start 127.486009 110.004089) (end 127.307227 110.482262) (stroke (width 0.05) (type default)) (layer "Edge.Cuts"))
 (gr_line (start 127.5623 103.481396) (end 127.875 103.680607) (stroke (width 0.05) (type default)) (layer "Edge.Cuts"))
 (gr_line (start 127.656418 109.522868) (end 127.486009 110.004089) (stroke (width 0.05) (type default)) (layer "Edge.Cuts"))
 (gr_line (start 127.818403 109.038747) (end 127.656418 109.522868) (stroke (width 0.05) (type default)) (layer "Edge.Cuts"))
 (gr_line (start 127.875 103.680607) (end 128.203871 103.851808) (stroke (width 0.05) (type default)) (layer "Edge.Cuts"))
 (gr_line (start 127.971914 108.551872) (end 127.818403 109.038747) (stroke (width 0.05) (type default)) (layer "Edge.Cuts"))
 (gr_line (start 128.116904 108.062392) (end 127.971914 108.551872) (stroke (width 0.05) (type default)) (layer "Edge.Cuts"))
 (gr_line (start 128.203871 103.851808) (end 128.546414 103.993693) (stroke (width 0.05) (type default)) (layer "Edge.Cuts"))
 (gr_line (start 128.25333 107.570457) (end 128.116904 108.062392) (stroke (width 0.05) (type default)) (layer "Edge.Cuts"))
 (gr_line (start 128.381149 107.076215) (end 128.25333 107.570457) (stroke (width 0.05) (type default)) (layer "Edge.Cuts"))
 (gr_line (start 128.500324 106.579818) (end 128.381149 107.076215) (stroke (width 0.05) (type default)) (layer "Edge.Cuts"))
 (gr_line (start 128.546414 103.993693) (end 128.900018 104.105184) (stroke (width 0.05) (type default)) (layer "Edge.Cuts"))
 (gr_line (start 128.610817 106.081416) (end 128.500324 106.579818) (stroke (width 0.05) (type default)) (layer "Edge.Cuts"))
 (gr_line (start 128.712595 105.581163) (end 128.610817 106.081416) (stroke (width 0.05) (type default)) (layer "Edge.Cuts"))
 (gr_line (start 128.805625 105.079209) (end 128.712595 105.581163) (stroke (width 0.05) (type default)) (layer "Edge.Cuts"))
 (gr_line (start 128.889883 104.575708) (end 128.805625 105.079209) (stroke (width 0.05) (type default)) (layer "Edge.Cuts"))
 (gr_line (start 128.900018 104.105184) (end 128.958273 104.118098) (stroke (width 0.05) (type default)) (layer "Edge.Cuts"))
 (gr_line (start 128.958273 104.118098) (end 128.889883 104.575708) (stroke (width 0.05) (type default)) (layer "Edge.Cuts"))
 (segment (start 113.48125 108.275) (end 116 108.275) (width 0.6) (layer "F.Cu") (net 1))
 (segment (start 116 108.275) (end 116.69573 107.805381) (width 0.6) (layer "F.Cu") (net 1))
 (segment (start 108.5 120.5) (end 108.5 110.1) (width 0.6) (layer "F.Cu") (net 1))
 (segment (start 117.367098 107.6) (end 126.4 107.6) (width 0.6) (layer "F.Cu") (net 1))
 (segment (start 113.2 108.61875) (end 113.2 108.55625) (width 0.6) (layer "F.Cu") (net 1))
 (segment (start 109.7 108.9) (end 112.91875 108.9) (width 0.6) (layer "F.Cu") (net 1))
 (arc (start 116.69573 107.805381) (mid 117.016058 107.652493) (end 117.367098 107.6) (width 0.6) (layer "F.Cu") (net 1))
 (arc (start 113.2 108.55625) (mid 113.282376 108.357376) (end 113.48125 108.275) (width 0.6) (layer "F.Cu") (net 1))
 (arc (start 108.5 110.1) (mid 108.851471 109.251471) (end 109.7 108.9) (width 0.6) (layer "F.Cu") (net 1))
 (arc (start 112.91875 108.9) (mid 113.117623 108.817623) (end 113.2 108.61875) (width 0.6) (layer "F.Cu") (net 1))
 (segment (start 113.2 113.5) (end 111.2 113.5) (width 0.6) (layer "F.Cu") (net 2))
 (segment (start 116 105.325) (end 124.864698 104.802082) (width 0.6) (layer "F.Cu") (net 2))
 (segment (start 124.935362 104.8) (end 126.4 104.8) (width 0.6) (layer "F.Cu") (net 2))
 (segment (start 109.325 123.04) (end 108.5 123.04) (width 0.6) (layer "F.Cu") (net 2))
 (segment (start 110 114.7) (end 110 122.365) (width 0.6) (layer "F.Cu") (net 2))
 (arc (start 124.864698 104.802082) (mid 124.900015 104.80052) (end 124.935362 104.8) (width 0.6) (layer "F.Cu") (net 2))
 (arc (start 110 122.365) (mid 109.802297 122.842297) (end 109.325 123.04) (width 0.6) (layer "F.Cu") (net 2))
 (arc (start 111.2 113.5) (mid 110.351471 113.851471) (end 110 114.7) (width 0.6) (layer "F.Cu") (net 2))
 (segment (start 112.7 102.8) (end 123.902943 102.8) (width 0.6) (layer "B.Cu") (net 2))
 (segment (start 108.5 123.04) (end 110.3 123.04) (width 0.6) (layer "B.Cu") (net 2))
 (segment (start 124.751471 103.151471) (end 126.4 104.8) (width 0.6) (layer "B.Cu") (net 2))
 (segment (start 111.5 121.84) (end 111.5 104) (width 0.6) (layer "B.Cu") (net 2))
 (arc (start 123.902943 102.8) (mid 124.362163 102.891344) (end 124.751471 103.151471) (width 0.6) (layer "B.Cu") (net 2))
 (arc (start 110.3 123.04) (mid 111.148528 122.688528) (end 111.5 121.84) (width 0.6) (layer "B.Cu") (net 2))
 (arc (start 111.5 104) (mid 111.851471 103.151471) (end 112.7 102.8) (width 0.6) (layer "B.Cu") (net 2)))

